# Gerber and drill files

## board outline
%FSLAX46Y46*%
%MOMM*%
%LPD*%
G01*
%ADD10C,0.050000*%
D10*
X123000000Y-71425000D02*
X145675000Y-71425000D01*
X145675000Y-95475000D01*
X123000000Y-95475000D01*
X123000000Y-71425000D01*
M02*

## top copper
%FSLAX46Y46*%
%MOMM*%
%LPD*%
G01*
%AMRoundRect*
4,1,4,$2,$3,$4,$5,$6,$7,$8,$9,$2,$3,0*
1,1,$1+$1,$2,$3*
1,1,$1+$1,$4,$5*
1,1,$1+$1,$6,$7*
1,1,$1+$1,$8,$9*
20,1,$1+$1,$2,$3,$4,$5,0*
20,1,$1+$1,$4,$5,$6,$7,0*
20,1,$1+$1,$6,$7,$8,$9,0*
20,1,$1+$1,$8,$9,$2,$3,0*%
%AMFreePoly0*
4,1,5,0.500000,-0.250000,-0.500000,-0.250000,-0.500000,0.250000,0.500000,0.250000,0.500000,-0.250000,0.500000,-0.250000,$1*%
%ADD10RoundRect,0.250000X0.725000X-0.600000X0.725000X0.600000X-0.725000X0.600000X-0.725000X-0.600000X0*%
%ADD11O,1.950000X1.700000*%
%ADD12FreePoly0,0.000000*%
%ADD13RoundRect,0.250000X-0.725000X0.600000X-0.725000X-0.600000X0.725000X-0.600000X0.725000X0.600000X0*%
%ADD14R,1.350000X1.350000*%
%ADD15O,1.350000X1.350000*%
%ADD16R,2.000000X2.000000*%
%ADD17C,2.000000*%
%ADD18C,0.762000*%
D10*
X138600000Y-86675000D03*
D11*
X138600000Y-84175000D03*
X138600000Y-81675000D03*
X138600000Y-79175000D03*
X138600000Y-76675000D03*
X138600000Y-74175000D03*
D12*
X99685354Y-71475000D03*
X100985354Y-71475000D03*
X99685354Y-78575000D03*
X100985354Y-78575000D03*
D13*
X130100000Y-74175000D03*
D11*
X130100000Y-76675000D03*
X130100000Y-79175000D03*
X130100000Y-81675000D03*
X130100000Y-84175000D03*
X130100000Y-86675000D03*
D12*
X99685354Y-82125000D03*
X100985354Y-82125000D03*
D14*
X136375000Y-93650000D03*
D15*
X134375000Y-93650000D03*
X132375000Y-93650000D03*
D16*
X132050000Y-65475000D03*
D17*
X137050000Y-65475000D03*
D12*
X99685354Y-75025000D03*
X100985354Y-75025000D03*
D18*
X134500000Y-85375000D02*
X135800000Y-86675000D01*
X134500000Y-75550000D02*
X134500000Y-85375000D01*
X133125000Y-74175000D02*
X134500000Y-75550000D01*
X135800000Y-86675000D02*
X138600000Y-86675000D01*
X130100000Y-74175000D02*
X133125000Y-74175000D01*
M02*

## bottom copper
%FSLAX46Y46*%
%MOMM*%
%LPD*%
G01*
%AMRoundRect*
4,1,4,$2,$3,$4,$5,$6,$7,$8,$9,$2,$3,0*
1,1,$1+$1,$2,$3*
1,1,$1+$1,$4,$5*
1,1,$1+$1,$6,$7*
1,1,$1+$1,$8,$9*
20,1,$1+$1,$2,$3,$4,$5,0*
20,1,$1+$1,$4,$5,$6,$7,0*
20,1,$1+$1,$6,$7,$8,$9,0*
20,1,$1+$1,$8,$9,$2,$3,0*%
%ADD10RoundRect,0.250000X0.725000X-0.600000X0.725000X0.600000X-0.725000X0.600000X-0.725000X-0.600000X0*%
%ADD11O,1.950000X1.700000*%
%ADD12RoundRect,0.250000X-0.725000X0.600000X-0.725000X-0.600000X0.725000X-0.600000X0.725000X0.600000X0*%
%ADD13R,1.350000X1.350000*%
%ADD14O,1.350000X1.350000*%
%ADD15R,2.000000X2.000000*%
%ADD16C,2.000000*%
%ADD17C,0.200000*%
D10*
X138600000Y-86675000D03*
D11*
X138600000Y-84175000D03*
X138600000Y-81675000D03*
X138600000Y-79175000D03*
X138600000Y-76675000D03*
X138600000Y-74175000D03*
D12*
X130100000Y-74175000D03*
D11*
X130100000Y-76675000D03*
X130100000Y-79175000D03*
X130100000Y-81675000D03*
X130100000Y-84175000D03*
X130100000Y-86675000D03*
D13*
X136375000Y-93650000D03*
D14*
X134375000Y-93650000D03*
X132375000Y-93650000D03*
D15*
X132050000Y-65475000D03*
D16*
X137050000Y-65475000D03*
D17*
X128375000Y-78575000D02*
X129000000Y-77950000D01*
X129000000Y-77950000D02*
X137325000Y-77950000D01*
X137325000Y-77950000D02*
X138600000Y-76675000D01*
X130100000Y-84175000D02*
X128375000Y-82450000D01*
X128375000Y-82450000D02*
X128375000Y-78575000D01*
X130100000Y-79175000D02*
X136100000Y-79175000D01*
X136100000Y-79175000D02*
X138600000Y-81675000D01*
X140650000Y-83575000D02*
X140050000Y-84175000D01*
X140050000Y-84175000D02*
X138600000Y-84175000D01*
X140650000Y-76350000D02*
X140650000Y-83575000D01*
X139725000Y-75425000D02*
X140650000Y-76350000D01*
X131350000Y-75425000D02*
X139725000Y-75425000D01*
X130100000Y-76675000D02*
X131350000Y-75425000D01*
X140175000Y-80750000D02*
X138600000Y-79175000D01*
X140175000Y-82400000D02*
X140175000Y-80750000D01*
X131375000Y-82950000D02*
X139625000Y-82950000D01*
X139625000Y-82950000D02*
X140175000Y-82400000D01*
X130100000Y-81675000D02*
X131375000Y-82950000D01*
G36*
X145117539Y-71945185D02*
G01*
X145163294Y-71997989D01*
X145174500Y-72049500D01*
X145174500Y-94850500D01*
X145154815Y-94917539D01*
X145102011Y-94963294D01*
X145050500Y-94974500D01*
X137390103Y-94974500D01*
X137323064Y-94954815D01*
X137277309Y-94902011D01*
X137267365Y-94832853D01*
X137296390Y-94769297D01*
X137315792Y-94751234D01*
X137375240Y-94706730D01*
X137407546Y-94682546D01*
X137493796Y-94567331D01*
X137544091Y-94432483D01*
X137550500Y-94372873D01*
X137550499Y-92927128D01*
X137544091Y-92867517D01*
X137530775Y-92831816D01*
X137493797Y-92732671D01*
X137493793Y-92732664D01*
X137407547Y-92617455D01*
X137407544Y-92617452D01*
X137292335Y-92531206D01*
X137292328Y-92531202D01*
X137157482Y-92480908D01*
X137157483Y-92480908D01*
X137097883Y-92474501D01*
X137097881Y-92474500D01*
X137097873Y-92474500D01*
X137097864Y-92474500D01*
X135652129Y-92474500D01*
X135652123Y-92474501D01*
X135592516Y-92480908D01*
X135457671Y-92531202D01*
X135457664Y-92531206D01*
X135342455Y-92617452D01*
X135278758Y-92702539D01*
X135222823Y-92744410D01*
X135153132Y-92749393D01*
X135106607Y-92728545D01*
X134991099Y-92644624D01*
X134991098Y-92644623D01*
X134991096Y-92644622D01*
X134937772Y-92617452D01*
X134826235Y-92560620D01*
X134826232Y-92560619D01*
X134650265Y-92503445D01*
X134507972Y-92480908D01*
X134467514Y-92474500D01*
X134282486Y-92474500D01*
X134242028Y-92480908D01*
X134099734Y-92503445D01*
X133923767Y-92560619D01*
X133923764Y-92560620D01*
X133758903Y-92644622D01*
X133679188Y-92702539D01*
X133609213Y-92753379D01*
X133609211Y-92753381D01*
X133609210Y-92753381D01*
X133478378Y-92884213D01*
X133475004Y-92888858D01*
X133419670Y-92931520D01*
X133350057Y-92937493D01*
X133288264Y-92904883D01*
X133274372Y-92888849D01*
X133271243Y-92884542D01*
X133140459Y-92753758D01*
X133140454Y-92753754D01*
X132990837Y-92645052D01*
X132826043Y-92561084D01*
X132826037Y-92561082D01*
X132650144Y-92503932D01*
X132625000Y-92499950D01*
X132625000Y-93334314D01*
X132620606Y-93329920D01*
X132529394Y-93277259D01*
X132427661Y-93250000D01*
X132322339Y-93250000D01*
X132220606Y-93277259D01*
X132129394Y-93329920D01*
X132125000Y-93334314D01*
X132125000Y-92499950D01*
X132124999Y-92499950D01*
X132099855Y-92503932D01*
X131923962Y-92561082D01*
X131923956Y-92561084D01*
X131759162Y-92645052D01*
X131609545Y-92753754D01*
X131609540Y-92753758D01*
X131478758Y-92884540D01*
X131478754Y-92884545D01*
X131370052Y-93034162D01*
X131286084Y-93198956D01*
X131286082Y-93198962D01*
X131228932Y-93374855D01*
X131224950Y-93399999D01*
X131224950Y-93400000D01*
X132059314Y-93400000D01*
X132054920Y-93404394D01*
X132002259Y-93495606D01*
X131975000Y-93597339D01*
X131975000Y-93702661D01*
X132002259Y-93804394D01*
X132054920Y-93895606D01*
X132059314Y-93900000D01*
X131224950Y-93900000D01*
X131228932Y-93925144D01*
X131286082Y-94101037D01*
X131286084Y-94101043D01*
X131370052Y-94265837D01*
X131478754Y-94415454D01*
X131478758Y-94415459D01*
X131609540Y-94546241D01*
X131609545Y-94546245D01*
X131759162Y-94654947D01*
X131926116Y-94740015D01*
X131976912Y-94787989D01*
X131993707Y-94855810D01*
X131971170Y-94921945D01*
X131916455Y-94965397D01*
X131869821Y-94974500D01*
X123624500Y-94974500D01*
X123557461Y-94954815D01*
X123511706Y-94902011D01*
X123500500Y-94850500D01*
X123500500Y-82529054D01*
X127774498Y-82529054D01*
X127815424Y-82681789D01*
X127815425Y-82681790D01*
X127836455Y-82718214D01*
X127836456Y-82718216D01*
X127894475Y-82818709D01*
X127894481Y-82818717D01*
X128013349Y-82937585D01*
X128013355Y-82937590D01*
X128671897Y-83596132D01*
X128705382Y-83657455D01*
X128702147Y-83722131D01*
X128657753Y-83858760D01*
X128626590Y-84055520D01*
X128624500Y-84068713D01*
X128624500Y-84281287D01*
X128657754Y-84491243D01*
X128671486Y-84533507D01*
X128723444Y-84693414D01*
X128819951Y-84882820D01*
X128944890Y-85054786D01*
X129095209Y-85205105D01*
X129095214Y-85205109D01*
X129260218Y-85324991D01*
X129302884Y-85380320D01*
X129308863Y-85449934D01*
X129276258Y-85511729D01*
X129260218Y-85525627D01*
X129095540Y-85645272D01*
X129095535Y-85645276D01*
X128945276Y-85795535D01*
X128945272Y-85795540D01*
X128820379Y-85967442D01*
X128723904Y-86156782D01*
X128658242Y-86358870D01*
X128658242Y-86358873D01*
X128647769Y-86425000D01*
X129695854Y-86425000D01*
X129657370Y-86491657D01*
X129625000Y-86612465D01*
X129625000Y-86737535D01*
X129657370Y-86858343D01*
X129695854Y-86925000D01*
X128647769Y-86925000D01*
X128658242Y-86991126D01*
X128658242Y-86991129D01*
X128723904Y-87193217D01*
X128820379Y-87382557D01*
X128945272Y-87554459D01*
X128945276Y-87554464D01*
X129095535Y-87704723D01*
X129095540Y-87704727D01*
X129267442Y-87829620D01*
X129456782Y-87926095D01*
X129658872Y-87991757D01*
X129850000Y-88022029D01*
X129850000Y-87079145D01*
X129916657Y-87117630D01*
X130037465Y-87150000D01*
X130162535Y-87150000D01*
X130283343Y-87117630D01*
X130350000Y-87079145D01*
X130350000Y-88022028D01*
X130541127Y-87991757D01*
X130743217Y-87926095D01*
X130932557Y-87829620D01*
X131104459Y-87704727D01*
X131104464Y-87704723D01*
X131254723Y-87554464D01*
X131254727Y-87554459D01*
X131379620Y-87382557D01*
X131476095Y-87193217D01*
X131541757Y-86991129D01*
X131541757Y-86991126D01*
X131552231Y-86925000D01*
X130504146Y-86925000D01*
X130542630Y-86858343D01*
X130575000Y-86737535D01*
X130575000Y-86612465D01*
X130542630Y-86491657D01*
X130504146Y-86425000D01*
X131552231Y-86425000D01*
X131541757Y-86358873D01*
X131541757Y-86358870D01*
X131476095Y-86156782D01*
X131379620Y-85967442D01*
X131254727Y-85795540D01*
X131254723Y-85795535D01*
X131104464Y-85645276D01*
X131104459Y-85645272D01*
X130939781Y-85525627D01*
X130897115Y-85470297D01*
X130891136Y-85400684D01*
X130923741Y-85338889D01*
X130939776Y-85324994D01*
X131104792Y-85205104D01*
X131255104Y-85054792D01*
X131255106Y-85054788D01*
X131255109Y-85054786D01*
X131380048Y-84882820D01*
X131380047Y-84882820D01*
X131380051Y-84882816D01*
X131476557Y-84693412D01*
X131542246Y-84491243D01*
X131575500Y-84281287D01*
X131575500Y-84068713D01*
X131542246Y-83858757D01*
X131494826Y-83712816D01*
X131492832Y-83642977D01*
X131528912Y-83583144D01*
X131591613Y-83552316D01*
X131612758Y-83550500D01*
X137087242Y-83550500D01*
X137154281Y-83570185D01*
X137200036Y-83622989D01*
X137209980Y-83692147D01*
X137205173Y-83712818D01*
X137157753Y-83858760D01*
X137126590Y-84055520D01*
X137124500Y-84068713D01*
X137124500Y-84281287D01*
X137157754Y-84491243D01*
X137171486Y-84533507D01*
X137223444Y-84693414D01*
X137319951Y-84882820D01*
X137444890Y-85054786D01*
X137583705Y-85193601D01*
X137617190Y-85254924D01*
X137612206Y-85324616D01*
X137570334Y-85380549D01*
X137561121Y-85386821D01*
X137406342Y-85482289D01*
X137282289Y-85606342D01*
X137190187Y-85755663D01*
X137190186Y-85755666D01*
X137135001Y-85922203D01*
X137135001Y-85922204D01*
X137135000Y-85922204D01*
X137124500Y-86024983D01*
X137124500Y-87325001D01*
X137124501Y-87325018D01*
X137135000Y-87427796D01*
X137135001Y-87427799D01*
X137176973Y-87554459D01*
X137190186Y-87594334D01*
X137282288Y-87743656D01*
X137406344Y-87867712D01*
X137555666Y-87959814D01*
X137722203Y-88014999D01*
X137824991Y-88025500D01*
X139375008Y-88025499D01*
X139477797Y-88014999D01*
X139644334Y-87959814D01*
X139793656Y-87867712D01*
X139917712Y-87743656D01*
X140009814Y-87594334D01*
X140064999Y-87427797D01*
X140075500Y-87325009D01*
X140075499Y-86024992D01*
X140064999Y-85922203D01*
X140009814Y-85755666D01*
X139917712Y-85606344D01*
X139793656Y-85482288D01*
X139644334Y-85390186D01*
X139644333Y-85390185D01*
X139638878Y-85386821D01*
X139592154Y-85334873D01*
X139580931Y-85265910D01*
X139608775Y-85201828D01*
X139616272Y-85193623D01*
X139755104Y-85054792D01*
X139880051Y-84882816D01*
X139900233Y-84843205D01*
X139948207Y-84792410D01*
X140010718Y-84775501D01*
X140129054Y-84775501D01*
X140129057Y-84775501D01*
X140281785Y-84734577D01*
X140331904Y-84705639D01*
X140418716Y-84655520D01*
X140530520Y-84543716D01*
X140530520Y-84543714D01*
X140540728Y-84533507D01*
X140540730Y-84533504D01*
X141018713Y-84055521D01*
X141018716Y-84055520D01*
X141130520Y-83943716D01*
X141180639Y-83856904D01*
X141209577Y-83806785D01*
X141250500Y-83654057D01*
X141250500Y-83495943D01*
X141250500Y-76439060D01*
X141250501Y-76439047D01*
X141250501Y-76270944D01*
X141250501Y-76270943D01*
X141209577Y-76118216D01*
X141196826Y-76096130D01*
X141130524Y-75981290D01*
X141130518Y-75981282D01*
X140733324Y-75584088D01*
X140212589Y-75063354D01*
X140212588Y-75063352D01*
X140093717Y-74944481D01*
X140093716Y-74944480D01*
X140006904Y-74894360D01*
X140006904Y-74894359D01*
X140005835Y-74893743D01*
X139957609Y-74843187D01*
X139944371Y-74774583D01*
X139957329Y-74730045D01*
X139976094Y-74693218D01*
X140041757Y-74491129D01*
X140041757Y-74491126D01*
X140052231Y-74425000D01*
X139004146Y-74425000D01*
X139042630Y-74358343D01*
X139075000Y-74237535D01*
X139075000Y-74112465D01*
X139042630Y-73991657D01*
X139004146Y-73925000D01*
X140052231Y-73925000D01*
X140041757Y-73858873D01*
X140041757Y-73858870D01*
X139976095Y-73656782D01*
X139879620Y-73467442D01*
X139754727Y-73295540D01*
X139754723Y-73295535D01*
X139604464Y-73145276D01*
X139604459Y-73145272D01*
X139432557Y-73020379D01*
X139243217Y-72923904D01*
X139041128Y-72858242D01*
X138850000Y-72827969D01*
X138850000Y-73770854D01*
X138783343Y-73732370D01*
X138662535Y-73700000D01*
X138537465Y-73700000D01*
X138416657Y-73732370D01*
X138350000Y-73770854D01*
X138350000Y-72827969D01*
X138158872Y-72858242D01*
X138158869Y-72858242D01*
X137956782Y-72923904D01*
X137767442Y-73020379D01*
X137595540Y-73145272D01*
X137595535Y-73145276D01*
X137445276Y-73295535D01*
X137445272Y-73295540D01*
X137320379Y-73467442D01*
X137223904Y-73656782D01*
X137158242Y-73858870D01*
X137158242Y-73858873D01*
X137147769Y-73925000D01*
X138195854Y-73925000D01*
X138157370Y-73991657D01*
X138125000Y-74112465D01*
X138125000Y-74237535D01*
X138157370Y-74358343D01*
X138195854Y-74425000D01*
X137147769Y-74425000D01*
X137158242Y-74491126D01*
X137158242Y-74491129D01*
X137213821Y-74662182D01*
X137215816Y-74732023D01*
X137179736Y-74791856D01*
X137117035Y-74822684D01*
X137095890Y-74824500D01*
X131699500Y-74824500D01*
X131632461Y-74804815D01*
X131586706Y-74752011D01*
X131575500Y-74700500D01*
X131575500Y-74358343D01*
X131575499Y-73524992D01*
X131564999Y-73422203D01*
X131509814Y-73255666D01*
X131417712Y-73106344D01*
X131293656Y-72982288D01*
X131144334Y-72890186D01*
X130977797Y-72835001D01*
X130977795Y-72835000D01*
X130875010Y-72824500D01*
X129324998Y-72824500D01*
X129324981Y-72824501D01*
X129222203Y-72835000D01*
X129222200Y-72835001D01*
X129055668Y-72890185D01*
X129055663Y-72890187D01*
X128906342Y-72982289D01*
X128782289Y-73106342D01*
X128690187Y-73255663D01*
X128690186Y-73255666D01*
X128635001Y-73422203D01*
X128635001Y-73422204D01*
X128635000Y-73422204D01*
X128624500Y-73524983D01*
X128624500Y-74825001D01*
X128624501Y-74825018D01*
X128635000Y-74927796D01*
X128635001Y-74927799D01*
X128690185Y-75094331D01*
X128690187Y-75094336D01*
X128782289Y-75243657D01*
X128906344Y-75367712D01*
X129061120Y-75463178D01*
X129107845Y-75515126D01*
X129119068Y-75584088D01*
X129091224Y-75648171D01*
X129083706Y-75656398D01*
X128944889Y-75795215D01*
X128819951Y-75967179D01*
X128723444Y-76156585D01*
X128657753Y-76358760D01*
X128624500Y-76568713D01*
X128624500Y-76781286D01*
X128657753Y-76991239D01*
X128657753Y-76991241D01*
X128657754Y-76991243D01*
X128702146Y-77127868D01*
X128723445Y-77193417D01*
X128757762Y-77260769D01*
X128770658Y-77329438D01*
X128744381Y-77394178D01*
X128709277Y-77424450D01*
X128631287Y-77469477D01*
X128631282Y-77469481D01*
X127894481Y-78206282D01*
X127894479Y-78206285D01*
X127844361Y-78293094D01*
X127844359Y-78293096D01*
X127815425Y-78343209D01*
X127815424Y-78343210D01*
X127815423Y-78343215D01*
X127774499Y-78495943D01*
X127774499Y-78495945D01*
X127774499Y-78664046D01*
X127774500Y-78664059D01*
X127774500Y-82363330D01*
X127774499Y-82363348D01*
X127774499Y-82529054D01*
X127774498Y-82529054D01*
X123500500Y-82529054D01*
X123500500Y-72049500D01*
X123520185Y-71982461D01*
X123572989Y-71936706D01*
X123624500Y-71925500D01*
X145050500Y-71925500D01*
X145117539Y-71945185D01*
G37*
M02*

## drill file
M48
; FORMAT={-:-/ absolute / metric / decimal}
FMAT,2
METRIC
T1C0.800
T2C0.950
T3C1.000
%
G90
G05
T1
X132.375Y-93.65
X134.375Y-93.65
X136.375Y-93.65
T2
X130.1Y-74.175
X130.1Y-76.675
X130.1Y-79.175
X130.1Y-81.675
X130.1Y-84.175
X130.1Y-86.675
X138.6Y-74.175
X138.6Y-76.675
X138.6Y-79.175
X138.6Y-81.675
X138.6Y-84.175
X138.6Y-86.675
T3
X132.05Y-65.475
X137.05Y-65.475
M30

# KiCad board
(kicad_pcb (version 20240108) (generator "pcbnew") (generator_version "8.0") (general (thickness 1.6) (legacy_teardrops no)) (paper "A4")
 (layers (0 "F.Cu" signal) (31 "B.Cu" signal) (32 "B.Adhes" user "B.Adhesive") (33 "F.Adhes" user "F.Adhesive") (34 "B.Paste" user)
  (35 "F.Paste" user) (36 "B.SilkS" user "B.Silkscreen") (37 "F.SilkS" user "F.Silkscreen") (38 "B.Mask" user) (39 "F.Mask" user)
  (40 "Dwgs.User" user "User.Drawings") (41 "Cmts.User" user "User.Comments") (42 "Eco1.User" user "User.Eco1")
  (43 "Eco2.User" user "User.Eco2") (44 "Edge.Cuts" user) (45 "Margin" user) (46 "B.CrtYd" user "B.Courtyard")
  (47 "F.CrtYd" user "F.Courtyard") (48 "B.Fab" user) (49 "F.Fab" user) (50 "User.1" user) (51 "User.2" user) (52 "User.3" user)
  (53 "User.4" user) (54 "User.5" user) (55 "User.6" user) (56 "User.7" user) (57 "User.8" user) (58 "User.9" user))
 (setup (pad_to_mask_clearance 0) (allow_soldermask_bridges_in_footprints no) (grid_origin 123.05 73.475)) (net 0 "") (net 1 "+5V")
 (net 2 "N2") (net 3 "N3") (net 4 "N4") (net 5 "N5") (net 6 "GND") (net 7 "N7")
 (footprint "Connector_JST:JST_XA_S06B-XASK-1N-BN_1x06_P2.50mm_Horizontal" (layer "F.Cu") (at 138.6 86.675 90)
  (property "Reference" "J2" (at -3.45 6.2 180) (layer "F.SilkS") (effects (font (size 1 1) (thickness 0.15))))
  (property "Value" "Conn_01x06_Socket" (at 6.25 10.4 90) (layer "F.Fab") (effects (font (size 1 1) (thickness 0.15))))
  (pad "1" thru_hole roundrect (at 0 0 90) (size 1.7 1.95) (drill 0.95) (layers "*.Cu" "*.Mask") (remove_unused_layers no)
   (roundrect_rratio 0.147059) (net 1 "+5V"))
  (pad "2" thru_hole oval (at 2.5 0 90) (size 1.7 1.95) (drill 0.95) (layers "*.Cu" "*.Mask") (remove_unused_layers no) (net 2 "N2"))
  (pad "3" thru_hole oval (at 5 0 90) (size 1.7 1.95) (drill 0.95) (layers "*.Cu" "*.Mask") (remove_unused_layers no) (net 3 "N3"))
  (pad "4" thru_hole oval (at 7.5 0 90) (size 1.7 1.95) (drill 0.95) (layers "*.Cu" "*.Mask") (remove_unused_layers no) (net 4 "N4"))
  (pad "5" thru_hole oval (at 10 0 90) (size 1.7 1.95) (drill 0.95) (layers "*.Cu" "*.Mask") (remove_unused_layers no) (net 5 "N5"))
  (pad "6" thru_hole oval (at 12.5 0 90) (size 1.7 1.95) (drill 0.95) (layers "*.Cu" "*.Mask") (remove_unused_layers no) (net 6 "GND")))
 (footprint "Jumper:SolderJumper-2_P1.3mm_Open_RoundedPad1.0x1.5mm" (layer "F.Cu") (at 100.335354 71.475)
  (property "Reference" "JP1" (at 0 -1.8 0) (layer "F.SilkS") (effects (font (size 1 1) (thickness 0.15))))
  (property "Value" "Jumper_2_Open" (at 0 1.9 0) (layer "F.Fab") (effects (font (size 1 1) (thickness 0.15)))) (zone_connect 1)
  (pad "1" smd custom (at -0.65 0) (size 1 0.5) (layers "F.Cu" "F.Mask") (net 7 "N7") (zone_connect 2) (thermal_bridge_angle 45)
   (options (clearance outline) (anchor rect)) (primitives))
  (pad "2" smd custom (at 0.65 0) (size 1 0.5) (layers "F.Cu" "F.Mask") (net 2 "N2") (zone_connect 2) (thermal_bridge_angle 45)
   (options (clearance outline) (anchor rect)) (primitives)))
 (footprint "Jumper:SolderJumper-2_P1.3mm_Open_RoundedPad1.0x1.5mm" (layer "F.Cu") (at 100.335354 78.575)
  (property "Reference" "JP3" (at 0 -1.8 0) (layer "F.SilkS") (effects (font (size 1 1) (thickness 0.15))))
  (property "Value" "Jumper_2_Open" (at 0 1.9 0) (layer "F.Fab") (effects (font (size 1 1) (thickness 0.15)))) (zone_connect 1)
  (pad "1" smd custom (at -0.65 0) (size 1 0.5) (layers "F.Cu" "F.Mask") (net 7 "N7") (zone_connect 2) (thermal_bridge_angle 45)
   (options (clearance outline) (anchor rect)) (primitives))
  (pad "2" smd custom (at 0.65 0) (size 1 0.5) (layers "F.Cu" "F.Mask") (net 4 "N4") (zone_connect 2) (thermal_bridge_angle 45)
   (options (clearance outline) (anchor rect)) (primitives)))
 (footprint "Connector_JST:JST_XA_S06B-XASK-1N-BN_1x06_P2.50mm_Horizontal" (layer "F.Cu") (at 130.1 74.175 -90)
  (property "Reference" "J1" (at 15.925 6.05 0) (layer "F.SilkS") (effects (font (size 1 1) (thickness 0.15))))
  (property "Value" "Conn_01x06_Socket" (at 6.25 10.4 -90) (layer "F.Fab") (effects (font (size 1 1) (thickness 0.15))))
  (pad "1" thru_hole roundrect (at 0 0 270) (size 1.7 1.95) (drill 0.95) (layers "*.Cu" "*.Mask") (remove_unused_layers no)
   (roundrect_rratio 0.147059) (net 1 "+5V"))
  (pad "2" thru_hole oval (at 2.5 0 270) (size 1.7 1.95) (drill 0.95) (layers "*.Cu" "*.Mask") (remove_unused_layers no) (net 2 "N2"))
  (pad "3" thru_hole oval (at 5 0 270) (size 1.7 1.95) (drill 0.95) (layers "*.Cu" "*.Mask") (remove_unused_layers no) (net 3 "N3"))
  (pad "4" thru_hole oval (at 7.5 0 270) (size 1.7 1.95) (drill 0.95) (layers "*.Cu" "*.Mask") (remove_unused_layers no) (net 4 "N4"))
  (pad "5" thru_hole oval (at 10 0 270) (size 1.7 1.95) (drill 0.95) (layers "*.Cu" "*.Mask") (remove_unused_layers no) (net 5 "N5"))
  (pad "6" thru_hole oval (at 12.5 0 270) (size 1.7 1.95) (drill 0.95) (layers "*.Cu" "*.Mask") (remove_unused_layers no) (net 6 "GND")))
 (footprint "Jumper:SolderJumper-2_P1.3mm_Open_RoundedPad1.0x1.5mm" (layer "F.Cu") (at 100.335354 82.125)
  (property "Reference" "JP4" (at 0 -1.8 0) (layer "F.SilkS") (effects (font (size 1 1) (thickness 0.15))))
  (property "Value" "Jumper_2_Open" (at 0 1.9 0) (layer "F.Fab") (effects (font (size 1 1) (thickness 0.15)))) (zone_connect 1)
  (pad "1" smd custom (at -0.65 0) (size 1 0.5) (layers "F.Cu" "F.Mask") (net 7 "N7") (zone_connect 2) (thermal_bridge_angle 45)
   (options (clearance outline) (anchor rect)) (primitives))
  (pad "2" smd custom (at 0.65 0) (size 1 0.5) (layers "F.Cu" "F.Mask") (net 5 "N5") (zone_connect 2) (thermal_bridge_angle 45)
   (options (clearance outline) (anchor rect)) (primitives)))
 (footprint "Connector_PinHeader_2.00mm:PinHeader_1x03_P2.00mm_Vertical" (layer "F.Cu") (at 136.375 93.65 -90)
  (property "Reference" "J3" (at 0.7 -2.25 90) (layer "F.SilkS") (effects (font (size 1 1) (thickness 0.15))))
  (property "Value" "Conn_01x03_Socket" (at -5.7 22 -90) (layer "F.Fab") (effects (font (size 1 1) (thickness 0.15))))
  (pad "1" thru_hole rect (at 0 0 270) (size 1.35 1.35) (drill 0.8) (layers "*.Cu" "*.Mask") (remove_unused_layers no) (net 1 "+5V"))
  (pad "2" thru_hole oval (at 0 2 270) (size 1.35 1.35) (drill 0.8) (layers "*.Cu" "*.Mask") (remove_unused_layers no) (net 7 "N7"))
  (pad "3" thru_hole oval (at 0 4 270) (size 1.35 1.35) (drill 0.8) (layers "*.Cu" "*.Mask") (remove_unused_layers no) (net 6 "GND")))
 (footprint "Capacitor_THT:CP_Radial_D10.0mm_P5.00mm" (layer "F.Cu") (at 132.05 65.475)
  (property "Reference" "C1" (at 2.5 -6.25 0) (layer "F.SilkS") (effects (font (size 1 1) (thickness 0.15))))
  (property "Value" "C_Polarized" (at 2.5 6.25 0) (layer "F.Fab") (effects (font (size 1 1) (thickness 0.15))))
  (pad "1" thru_hole rect (at 0 0) (size 2 2) (drill 1) (layers "*.Cu" "*.Mask") (remove_unused_layers no) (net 1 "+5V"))
  (pad "2" thru_hole circle (at 5 0) (size 2 2) (drill 1) (layers "*.Cu" "*.Mask") (remove_unused_layers no) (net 6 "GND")))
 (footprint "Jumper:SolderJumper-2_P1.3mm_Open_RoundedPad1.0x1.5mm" (layer "F.Cu") (at 100.335354 75.025)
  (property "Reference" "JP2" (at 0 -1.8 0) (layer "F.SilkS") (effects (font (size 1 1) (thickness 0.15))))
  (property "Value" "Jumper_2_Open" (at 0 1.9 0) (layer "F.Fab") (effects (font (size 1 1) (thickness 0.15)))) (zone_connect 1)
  (pad "1" smd custom (at -0.65 0) (size 1 0.5) (layers "F.Cu" "F.Mask") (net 7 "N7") (zone_connect 2) (thermal_bridge_angle 45)
   (options (clearance outline) (anchor rect)) (primitives))
  (pad "2" smd custom (at 0.65 0) (size 1 0.5) (layers "F.Cu" "F.Mask") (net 3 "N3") (zone_connect 2) (thermal_bridge_angle 45)
   (options (clearance outline) (anchor rect)) (primitives)))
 (gr_rect (start 123 71.425) (end 145.675 95.475) (stroke (width 0.05) (type default)) (fill none) (layer "Edge.Cuts"))
 (segment (start 134.5 85.375) (end 135.8 86.675) (width 0.762) (layer "F.Cu") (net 1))
 (segment (start 134.5 75.55) (end 134.5 85.375) (width 0.762) (layer "F.Cu") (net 1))
 (segment (start 133.125 74.175) (end 134.5 75.55) (width 0.762) (layer "F.Cu") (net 1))
 (segment (start 135.8 86.675) (end 138.6 86.675) (width 0.762) (layer "F.Cu") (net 1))
 (segment (start 130.1 74.175) (end 133.125 74.175) (width 0.762) (layer "F.Cu") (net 1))
 (segment (start 128.375 78.575) (end 129 77.95) (width 0.2) (layer "B.Cu") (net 5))
 (segment (start 129 77.95) (end 137.325 77.95) (width 0.2) (layer "B.Cu") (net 5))
 (segment (start 137.325 77.95) (end 138.6 76.675) (width 0.2) (layer "B.Cu") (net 5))
 (segment (start 130.1 84.175) (end 128.375 82.45) (width 0.2) (layer "B.Cu") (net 5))
 (segment (start 128.375 82.45) (end 128.375 78.575) (width 0.2) (layer "B.Cu") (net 5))
 (segment (start 130.1 79.175) (end 136.1 79.175) (width 0.2) (layer "B.Cu") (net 3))
 (segment (start 136.1 79.175) (end 138.6 81.675) (width 0.2) (layer "B.Cu") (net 3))
 (segment (start 140.65 83.575) (end 140.05 84.175) (width 0.2) (layer "B.Cu") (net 2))
 (segment (start 140.05 84.175) (end 138.6 84.175) (width 0.2) (layer "B.Cu") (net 2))
 (segment (start 140.65 76.35) (end 140.65 83.575) (width 0.2) (layer "B.Cu") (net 2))
 (segment (start 139.725 75.425) (end 140.65 76.35) (width 0.2) (layer "B.Cu") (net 2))
 (segment (start 131.35 75.425) (end 139.725 75.425) (width 0.2) (layer "B.Cu") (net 2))
 (segment (start 130.1 76.675) (end 131.35 75.425) (width 0.2) (layer "B.Cu") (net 2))
 (segment (start 140.175 80.75) (end 138.6 79.175) (width 0.2) (layer "B.Cu") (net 4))
 (segment (start 140.175 82.4) (end 140.175 80.75) (width 0.2) (layer "B.Cu") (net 4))
 (segment (start 131.375 82.95) (end 139.625 82.95) (width 0.2) (layer "B.Cu") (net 4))
 (segment (start 139.625 82.95) (end 140.175 82.4) (width 0.2) (layer "B.Cu") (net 4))
 (segment (start 130.1 81.675) (end 131.375 82.95) (width 0.2) (layer "B.Cu") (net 4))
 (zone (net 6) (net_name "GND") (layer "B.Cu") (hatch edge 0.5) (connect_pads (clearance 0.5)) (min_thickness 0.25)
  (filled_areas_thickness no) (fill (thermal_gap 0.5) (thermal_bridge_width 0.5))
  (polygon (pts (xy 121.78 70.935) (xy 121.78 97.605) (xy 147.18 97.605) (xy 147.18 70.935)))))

